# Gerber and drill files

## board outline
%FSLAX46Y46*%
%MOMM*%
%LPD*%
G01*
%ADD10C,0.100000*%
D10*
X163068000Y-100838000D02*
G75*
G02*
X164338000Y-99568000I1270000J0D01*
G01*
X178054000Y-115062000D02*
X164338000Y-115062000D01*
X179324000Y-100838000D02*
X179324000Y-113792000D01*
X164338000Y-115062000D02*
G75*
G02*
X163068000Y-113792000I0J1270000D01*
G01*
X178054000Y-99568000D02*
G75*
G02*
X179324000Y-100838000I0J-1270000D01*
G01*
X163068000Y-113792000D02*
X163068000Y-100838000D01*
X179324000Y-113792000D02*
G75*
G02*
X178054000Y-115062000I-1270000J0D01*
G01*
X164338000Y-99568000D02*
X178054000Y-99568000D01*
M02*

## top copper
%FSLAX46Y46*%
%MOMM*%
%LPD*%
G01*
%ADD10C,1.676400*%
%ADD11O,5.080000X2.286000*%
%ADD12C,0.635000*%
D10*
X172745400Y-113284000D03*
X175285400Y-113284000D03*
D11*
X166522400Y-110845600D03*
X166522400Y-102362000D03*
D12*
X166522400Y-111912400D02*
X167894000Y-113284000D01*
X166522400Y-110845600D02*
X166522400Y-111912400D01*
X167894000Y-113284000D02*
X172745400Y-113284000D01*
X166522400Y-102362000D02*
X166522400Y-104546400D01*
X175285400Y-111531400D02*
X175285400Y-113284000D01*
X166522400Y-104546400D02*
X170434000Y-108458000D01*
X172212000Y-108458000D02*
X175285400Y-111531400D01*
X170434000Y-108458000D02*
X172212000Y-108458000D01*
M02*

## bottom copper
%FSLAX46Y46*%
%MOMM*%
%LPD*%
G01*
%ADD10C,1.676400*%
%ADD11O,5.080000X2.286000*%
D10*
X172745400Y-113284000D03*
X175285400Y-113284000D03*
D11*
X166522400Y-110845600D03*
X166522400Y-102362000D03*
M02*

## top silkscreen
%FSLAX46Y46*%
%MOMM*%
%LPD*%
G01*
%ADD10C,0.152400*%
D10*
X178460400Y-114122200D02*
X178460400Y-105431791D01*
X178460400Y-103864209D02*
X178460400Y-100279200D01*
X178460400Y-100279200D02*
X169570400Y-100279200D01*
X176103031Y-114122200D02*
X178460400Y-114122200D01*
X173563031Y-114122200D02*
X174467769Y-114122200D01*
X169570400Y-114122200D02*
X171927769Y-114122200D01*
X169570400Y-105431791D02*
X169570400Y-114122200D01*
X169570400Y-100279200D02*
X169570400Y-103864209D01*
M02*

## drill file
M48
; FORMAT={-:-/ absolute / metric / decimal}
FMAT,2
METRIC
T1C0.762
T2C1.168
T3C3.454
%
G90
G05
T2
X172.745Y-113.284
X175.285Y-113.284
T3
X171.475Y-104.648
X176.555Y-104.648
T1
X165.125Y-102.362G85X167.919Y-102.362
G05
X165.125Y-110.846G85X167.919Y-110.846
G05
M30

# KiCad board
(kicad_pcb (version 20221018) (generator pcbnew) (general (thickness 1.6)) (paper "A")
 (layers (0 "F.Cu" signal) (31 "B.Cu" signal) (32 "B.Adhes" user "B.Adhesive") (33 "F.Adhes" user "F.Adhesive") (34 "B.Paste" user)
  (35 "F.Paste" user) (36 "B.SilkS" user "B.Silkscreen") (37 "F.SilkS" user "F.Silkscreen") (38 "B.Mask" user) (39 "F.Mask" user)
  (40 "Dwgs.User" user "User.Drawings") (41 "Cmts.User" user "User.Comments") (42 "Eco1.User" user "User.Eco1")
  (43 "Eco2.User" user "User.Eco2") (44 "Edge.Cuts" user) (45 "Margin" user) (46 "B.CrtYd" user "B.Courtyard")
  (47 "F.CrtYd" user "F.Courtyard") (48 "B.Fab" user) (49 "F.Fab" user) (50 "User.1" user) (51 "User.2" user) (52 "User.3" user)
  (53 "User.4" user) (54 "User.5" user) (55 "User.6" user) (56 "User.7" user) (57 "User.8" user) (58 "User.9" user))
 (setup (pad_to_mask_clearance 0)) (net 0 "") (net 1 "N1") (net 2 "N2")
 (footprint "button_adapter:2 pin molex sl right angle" (layer "F.Cu") (at 172.7454 113.284 180)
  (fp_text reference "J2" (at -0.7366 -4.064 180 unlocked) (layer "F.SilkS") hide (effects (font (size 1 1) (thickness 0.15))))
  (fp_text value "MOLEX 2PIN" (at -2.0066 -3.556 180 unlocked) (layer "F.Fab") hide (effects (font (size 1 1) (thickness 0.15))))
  (fp_line (start -5.715 -0.8382) (end -5.715 7.852209) (stroke (width 0.1524) (type solid)) (layer "F.SilkS"))
  (fp_line (start -5.715 9.419791) (end -5.715 13.0048) (stroke (width 0.1524) (type solid)) (layer "F.SilkS"))
  (fp_line (start -5.715 13.0048) (end 3.175 13.0048) (stroke (width 0.1524) (type solid)) (layer "F.SilkS"))
  (fp_line (start -3.357631 -0.8382) (end -5.715 -0.8382) (stroke (width 0.1524) (type solid)) (layer "F.SilkS"))
  (fp_line (start -0.817631 -0.8382) (end -1.722369 -0.8382) (stroke (width 0.1524) (type solid)) (layer "F.SilkS"))
  (fp_line (start 3.175 -0.8382) (end 0.817631 -0.8382) (stroke (width 0.1524) (type solid)) (layer "F.SilkS"))
  (fp_line (start 3.175 7.852209) (end 3.175 -0.8382) (stroke (width 0.1524) (type solid)) (layer "F.SilkS"))
  (fp_line (start 3.175 13.0048) (end 3.175 9.419791) (stroke (width 0.1524) (type solid)) (layer "F.SilkS"))
  (pad "" np_thru_hole circle (at -3.81 8.636 180) (size 3.4544 3.4544) (drill 3.4544) (layers))
  (pad "" np_thru_hole circle (at 1.27 8.636 180) (size 3.4544 3.4544) (drill 3.4544) (layers))
  (pad "1" thru_hole circle (at 0 0 180) (size 1.6764 1.6764) (drill 1.1684) (layers "*.Cu" "*.Mask") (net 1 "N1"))
  (pad "2" thru_hole circle (at -2.54 0 180) (size 1.6764 1.6764) (drill 1.1684) (layers "*.Cu" "*.Mask") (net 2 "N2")))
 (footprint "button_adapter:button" (layer "B.Cu") (at 166.5224 106.6038 90)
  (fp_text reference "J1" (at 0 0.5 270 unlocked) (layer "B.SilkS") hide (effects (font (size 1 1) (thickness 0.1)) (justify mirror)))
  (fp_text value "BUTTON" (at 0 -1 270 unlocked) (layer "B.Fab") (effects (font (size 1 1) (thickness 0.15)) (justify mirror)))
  (pad "1" thru_hole oval (at -4.2418 0 90) (size 2.286 5.08) (drill oval 0.762 3.556) (layers "*.Cu" "*.Mask") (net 1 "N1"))
  (pad "2" thru_hole oval (at 4.2418 0 90) (size 2.286 5.08) (drill oval 0.762 3.556) (layers "*.Cu" "*.Mask") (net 2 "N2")))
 (gr_arc (start 163.068 100.838) (mid 163.439974 99.939974) (end 164.338 99.568) (stroke (width 0.1) (type default)) (layer "Edge.Cuts"))
 (gr_line (start 178.054 115.062) (end 164.338 115.062) (stroke (width 0.1) (type default)) (layer "Edge.Cuts"))
 (gr_line (start 179.324 100.838) (end 179.324 113.792) (stroke (width 0.1) (type default)) (layer "Edge.Cuts"))
 (gr_arc (start 164.338 115.062) (mid 163.439974 114.690026) (end 163.068 113.792) (stroke (width 0.1) (type default)) (layer "Edge.Cuts"))
 (gr_arc (start 178.054 99.568) (mid 178.952026 99.939974) (end 179.324 100.838) (stroke (width 0.1) (type default)) (layer "Edge.Cuts"))
 (gr_line (start 163.068 113.792) (end 163.068 100.838) (stroke (width 0.1) (type default)) (layer "Edge.Cuts"))
 (gr_arc (start 179.324 113.792) (mid 178.952026 114.690026) (end 178.054 115.062) (stroke (width 0.1) (type default)) (layer "Edge.Cuts"))
 (gr_line (start 164.338 99.568) (end 178.054 99.568) (stroke (width 0.1) (type default)) (layer "Edge.Cuts"))
 (segment (start 166.5224 111.9124) (end 167.894 113.284) (width 0.635) (layer "F.Cu") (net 1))
 (segment (start 166.5224 110.8456) (end 166.5224 111.9124) (width 0.635) (layer "F.Cu") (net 1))
 (segment (start 167.894 113.284) (end 172.7454 113.284) (width 0.635) (layer "F.Cu") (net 1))
 (segment (start 166.5224 102.362) (end 166.5224 104.5464) (width 0.635) (layer "F.Cu") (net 2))
 (segment (start 175.2854 111.5314) (end 175.2854 113.284) (width 0.635) (layer "F.Cu") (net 2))
 (segment (start 166.5224 104.5464) (end 170.434 108.458) (width 0.635) (layer "F.Cu") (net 2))
 (segment (start 172.212 108.458) (end 175.2854 111.5314) (width 0.635) (layer "F.Cu") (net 2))
 (segment (start 170.434 108.458) (end 172.212 108.458) (width 0.635) (layer "F.Cu") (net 2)))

